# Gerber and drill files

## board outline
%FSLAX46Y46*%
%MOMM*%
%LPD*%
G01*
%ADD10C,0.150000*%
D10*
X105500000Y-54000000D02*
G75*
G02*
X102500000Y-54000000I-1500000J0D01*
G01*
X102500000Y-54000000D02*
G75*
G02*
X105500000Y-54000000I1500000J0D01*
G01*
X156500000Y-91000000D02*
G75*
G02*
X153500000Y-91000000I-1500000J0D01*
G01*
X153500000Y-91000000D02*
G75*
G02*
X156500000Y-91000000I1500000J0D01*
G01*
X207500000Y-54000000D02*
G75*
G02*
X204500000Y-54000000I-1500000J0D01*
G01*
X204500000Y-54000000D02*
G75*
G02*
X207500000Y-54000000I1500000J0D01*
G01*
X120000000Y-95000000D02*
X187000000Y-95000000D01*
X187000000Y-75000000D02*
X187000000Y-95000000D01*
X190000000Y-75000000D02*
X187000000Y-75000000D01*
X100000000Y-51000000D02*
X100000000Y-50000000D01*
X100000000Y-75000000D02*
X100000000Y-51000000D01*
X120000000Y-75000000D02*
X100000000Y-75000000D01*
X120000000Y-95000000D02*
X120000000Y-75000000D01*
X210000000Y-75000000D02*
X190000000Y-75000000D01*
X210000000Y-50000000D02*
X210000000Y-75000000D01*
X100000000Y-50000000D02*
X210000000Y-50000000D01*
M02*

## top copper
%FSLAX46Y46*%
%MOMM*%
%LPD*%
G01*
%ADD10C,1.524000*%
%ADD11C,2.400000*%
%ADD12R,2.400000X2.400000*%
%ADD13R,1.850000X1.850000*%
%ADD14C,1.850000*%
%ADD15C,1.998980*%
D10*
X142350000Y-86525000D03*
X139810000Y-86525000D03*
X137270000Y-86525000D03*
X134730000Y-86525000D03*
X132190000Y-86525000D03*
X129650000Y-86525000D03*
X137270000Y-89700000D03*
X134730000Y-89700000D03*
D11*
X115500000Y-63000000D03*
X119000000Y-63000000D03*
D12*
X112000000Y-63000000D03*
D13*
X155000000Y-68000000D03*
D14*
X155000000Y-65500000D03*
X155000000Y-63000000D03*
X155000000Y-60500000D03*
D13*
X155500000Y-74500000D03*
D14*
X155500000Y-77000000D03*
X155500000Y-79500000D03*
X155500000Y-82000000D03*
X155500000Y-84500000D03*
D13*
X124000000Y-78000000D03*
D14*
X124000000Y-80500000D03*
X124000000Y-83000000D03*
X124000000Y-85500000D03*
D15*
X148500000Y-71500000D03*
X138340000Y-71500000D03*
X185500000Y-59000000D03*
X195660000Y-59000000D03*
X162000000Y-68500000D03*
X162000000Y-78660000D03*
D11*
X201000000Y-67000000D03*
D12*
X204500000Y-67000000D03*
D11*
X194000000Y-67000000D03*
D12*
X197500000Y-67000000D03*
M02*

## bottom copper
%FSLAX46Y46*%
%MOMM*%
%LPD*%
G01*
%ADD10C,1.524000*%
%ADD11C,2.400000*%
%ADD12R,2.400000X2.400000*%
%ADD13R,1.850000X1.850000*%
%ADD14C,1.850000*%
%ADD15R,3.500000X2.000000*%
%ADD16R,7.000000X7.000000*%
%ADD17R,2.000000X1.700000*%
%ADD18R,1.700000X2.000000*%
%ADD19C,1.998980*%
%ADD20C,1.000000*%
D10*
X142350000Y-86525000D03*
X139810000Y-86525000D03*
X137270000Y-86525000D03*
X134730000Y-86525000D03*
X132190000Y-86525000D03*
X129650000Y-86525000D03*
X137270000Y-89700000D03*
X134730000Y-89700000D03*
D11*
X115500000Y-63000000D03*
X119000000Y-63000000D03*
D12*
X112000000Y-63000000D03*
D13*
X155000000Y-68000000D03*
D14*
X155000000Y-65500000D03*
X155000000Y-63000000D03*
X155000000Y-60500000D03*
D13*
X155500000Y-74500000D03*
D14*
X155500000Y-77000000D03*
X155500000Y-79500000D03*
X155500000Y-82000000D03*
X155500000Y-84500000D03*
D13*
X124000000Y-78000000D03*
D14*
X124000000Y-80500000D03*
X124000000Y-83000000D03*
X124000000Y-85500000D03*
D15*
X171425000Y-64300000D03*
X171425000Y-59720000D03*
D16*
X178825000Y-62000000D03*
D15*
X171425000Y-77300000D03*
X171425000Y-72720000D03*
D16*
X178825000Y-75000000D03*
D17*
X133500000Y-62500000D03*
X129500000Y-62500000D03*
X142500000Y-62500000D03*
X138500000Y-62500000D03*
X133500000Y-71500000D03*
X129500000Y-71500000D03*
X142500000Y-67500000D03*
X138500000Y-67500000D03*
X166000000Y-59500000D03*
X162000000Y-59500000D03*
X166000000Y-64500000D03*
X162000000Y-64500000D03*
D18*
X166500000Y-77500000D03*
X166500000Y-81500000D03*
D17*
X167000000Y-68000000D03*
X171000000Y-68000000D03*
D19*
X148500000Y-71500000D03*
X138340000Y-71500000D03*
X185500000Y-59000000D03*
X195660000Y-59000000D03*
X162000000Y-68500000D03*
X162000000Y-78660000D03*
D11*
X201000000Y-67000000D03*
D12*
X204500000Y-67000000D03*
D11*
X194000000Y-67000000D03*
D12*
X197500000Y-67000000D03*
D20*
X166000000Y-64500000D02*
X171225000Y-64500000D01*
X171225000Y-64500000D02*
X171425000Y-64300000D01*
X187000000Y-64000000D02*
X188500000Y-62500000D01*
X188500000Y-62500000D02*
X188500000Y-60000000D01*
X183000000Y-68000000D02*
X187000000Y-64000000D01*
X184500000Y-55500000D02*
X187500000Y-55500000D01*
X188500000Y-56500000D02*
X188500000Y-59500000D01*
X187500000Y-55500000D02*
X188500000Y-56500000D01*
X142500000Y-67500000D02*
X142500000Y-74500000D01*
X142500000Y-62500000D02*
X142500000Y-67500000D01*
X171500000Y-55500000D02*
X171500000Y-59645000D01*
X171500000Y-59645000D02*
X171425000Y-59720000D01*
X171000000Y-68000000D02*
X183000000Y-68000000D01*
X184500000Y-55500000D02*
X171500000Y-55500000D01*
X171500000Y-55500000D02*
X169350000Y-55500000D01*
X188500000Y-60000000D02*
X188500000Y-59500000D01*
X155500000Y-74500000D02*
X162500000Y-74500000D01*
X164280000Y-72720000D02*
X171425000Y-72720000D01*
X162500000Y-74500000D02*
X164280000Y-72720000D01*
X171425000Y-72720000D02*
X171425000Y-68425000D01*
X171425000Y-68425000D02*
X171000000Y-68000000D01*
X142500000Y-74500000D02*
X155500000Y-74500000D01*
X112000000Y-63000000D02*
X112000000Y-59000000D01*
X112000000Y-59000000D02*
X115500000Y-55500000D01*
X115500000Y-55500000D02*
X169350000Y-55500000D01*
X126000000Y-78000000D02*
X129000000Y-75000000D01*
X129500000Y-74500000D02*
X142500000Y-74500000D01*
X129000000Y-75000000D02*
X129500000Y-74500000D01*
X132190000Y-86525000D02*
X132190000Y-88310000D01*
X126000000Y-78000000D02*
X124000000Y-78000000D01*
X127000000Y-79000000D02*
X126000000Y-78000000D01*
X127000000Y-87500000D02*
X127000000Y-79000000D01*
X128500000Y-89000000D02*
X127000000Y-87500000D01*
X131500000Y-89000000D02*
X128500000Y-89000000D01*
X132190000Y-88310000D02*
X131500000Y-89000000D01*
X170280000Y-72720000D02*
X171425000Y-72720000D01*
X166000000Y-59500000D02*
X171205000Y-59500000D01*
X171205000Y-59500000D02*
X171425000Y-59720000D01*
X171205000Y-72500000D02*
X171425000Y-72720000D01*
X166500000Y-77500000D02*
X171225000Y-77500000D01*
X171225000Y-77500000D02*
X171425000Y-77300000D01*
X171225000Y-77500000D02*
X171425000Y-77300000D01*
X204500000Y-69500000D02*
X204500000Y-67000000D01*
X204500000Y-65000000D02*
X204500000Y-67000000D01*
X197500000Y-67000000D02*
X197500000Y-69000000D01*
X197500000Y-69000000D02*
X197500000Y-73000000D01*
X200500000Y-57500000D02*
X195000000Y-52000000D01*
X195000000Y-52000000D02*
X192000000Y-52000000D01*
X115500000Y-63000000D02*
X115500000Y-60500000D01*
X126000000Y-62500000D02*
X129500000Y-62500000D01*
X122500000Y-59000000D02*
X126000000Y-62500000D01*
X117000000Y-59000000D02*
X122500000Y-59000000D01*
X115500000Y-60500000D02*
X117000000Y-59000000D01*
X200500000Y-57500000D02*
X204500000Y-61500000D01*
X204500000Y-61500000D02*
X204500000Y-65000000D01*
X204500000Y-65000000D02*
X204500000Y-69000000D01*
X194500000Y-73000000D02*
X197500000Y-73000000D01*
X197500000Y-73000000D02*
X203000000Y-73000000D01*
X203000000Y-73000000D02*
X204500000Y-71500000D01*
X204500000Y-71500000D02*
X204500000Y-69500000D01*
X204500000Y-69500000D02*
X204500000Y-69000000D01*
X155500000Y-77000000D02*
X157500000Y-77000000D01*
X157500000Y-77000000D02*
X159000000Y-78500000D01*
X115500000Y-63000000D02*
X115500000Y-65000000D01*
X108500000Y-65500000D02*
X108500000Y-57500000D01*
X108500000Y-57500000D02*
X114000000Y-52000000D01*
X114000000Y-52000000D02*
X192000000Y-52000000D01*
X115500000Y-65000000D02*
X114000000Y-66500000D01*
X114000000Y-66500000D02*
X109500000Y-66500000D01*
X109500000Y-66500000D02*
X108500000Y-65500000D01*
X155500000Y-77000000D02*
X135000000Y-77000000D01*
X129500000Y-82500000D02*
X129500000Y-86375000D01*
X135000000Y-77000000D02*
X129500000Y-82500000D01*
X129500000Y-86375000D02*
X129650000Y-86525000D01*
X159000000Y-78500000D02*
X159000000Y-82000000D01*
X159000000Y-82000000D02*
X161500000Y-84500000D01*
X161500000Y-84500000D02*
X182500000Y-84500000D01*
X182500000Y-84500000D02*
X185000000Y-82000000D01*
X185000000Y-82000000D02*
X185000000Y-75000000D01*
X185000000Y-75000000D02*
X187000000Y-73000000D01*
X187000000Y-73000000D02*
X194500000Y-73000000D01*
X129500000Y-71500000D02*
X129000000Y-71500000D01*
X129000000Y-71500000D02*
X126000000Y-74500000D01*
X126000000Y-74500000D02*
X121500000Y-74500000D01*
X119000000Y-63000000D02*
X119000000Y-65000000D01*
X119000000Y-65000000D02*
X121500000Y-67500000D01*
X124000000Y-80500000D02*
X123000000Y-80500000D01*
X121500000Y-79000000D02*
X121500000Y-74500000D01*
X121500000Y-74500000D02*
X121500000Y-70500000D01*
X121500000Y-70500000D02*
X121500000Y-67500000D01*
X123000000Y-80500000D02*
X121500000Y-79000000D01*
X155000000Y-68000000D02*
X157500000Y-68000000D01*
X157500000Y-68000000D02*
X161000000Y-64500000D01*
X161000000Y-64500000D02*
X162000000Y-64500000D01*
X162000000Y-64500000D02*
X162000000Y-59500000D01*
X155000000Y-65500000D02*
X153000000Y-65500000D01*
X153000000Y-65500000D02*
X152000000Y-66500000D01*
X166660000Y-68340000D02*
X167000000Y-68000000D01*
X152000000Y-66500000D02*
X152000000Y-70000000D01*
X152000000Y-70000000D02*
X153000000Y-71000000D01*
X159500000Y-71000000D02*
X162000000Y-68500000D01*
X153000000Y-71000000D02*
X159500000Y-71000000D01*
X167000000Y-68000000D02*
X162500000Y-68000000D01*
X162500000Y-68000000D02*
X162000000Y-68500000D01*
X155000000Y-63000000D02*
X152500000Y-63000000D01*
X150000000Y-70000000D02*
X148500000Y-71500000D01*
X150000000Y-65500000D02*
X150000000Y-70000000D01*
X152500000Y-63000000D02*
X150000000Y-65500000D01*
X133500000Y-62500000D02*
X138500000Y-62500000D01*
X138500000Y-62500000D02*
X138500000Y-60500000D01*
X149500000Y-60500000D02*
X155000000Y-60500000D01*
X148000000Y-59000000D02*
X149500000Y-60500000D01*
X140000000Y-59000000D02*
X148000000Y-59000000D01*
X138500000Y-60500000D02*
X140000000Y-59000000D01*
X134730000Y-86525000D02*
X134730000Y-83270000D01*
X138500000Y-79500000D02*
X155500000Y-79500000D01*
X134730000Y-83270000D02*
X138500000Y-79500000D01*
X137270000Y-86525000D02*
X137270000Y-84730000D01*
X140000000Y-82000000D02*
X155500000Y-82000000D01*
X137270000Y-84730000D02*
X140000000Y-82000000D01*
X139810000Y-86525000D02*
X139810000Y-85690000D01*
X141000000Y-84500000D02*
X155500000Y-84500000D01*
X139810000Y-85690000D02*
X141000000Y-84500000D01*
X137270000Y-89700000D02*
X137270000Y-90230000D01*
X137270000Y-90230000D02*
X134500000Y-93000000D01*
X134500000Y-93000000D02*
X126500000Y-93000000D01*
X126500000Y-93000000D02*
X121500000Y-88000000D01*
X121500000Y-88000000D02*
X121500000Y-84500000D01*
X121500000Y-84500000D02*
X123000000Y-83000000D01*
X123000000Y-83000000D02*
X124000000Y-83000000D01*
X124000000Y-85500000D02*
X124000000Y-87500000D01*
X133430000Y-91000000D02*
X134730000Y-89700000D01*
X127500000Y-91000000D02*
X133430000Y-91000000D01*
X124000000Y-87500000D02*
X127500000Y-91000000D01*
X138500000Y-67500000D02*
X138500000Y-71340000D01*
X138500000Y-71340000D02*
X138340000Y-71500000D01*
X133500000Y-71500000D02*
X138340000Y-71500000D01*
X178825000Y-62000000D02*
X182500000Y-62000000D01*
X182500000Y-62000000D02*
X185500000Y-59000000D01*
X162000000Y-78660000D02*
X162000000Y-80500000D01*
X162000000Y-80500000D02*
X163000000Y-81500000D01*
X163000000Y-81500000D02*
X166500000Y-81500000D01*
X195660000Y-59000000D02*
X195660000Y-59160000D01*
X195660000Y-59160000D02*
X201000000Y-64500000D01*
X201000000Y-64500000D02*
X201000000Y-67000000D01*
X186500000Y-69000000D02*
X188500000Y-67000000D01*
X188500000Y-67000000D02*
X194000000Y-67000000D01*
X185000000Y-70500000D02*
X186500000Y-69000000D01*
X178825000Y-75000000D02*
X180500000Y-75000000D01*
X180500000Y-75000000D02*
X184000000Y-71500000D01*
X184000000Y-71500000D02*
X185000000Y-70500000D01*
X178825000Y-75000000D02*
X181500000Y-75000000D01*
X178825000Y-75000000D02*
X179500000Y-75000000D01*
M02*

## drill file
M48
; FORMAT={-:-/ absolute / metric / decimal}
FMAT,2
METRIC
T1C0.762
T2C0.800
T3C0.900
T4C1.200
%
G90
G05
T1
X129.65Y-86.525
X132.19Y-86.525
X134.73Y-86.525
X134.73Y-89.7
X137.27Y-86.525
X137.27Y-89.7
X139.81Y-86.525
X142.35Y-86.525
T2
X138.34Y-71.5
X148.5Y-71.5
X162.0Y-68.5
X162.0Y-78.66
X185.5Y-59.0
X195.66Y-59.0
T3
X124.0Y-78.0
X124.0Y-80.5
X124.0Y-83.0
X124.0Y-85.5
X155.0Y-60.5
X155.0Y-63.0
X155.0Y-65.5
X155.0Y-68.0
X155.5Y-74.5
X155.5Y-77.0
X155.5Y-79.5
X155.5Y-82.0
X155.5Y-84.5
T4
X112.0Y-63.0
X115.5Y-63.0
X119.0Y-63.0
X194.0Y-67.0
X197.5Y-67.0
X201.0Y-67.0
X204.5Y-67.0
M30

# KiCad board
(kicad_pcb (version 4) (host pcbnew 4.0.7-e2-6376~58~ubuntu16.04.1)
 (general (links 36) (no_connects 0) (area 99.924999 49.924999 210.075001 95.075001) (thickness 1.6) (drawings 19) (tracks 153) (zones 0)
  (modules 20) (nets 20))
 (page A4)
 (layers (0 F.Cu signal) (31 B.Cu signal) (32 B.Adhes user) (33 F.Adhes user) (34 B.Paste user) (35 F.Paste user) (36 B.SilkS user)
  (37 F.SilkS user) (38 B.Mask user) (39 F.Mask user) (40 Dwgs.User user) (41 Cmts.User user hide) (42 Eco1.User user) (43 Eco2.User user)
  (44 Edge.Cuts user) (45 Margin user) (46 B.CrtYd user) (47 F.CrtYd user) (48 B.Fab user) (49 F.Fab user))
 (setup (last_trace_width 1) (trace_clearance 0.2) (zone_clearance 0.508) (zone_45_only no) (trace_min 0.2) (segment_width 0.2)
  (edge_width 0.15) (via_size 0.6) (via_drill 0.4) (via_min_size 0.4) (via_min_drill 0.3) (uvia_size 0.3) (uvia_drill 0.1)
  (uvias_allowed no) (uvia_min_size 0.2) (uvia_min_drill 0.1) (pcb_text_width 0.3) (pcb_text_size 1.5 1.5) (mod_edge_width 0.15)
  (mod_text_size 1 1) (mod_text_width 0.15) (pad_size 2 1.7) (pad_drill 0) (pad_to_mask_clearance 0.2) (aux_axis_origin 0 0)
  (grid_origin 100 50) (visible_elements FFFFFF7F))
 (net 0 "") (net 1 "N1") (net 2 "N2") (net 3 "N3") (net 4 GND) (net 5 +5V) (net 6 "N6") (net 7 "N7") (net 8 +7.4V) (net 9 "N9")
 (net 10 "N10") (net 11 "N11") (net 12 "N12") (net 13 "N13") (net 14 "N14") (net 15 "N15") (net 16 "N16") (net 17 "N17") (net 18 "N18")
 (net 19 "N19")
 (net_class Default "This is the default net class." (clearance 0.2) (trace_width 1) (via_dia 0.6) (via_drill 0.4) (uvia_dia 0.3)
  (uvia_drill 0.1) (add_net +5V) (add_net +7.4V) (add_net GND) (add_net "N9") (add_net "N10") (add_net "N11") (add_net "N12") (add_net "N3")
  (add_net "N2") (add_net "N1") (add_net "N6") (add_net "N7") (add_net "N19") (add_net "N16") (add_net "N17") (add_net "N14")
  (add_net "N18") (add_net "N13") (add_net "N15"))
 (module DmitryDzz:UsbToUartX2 (layer F.Cu) (at 136 77)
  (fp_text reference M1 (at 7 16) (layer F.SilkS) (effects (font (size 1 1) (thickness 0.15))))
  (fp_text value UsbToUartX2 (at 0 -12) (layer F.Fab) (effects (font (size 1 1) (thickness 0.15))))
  (pad 1 thru_hole circle (at 6.35 9.525) (size 1.524 1.524) (drill 0.762) (layers *.Cu *.Mask))
  (pad 2 thru_hole circle (at 3.81 9.525) (size 1.524 1.524) (drill 0.762) (layers *.Cu *.Mask) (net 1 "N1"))
  (pad 3 thru_hole circle (at 1.27 9.525) (size 1.524 1.524) (drill 0.762) (layers *.Cu *.Mask) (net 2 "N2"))
  (pad 4 thru_hole circle (at -1.27 9.525) (size 1.524 1.524) (drill 0.762) (layers *.Cu *.Mask) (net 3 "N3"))
  (pad 5 thru_hole circle (at -3.81 9.525) (size 1.524 1.524) (drill 0.762) (layers *.Cu *.Mask) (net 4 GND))
  (pad 6 thru_hole circle (at -6.35 9.525) (size 1.524 1.524) (drill 0.762) (layers *.Cu *.Mask) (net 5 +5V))
  (pad 7 thru_hole circle (at 1.27 12.7) (size 1.524 1.524) (drill 0.762) (layers *.Cu *.Mask) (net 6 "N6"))
  (pad 8 thru_hole circle (at -1.27 12.7) (size 1.524 1.524) (drill 0.762) (layers *.Cu *.Mask) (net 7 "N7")))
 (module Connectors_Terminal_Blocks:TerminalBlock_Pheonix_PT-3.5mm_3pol (layer F.Cu) (at 112 63)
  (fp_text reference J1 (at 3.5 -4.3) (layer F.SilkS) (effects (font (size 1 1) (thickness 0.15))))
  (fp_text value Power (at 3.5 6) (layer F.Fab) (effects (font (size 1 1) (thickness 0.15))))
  (pad 2 thru_hole circle (at 3.5 0) (size 2.4 2.4) (drill 1.2) (layers *.Cu *.Mask) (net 5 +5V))
  (pad 3 thru_hole circle (at 7 0) (size 2.4 2.4) (drill 1.2) (layers *.Cu *.Mask) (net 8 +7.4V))
  (pad 1 thru_hole rect (at 0 0) (size 2.4 2.4) (drill 1.2) (layers *.Cu *.Mask) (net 4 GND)))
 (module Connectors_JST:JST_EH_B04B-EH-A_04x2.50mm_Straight (layer F.Cu) (at 155 68 90)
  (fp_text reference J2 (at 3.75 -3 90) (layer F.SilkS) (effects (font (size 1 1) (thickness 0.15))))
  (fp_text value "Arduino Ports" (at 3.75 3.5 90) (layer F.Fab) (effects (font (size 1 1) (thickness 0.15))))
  (pad 1 thru_hole rect (at 0 0 90) (size 1.85 1.85) (drill 0.9) (layers *.Cu *.Mask) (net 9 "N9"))
  (pad 2 thru_hole circle (at 2.5 0 90) (size 1.85 1.85) (drill 0.9) (layers *.Cu *.Mask) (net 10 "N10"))
  (pad 3 thru_hole circle (at 5 0 90) (size 1.85 1.85) (drill 0.9) (layers *.Cu *.Mask) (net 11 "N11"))
  (pad 4 thru_hole circle (at 7.5 0 90) (size 1.85 1.85) (drill 0.9) (layers *.Cu *.Mask) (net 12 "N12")))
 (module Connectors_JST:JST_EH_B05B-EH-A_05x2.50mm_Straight (layer F.Cu) (at 155.5 74.5 270)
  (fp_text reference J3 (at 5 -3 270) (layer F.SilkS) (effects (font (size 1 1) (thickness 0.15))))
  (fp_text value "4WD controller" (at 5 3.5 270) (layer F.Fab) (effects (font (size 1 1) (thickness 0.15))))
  (pad 1 thru_hole rect (at 0 0 270) (size 1.85 1.85) (drill 0.9) (layers *.Cu *.Mask) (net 4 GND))
  (pad 2 thru_hole circle (at 2.5 0 270) (size 1.85 1.85) (drill 0.9) (layers *.Cu *.Mask) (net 5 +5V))
  (pad 3 thru_hole circle (at 5 0 270) (size 1.85 1.85) (drill 0.9) (layers *.Cu *.Mask) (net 3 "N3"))
  (pad 4 thru_hole circle (at 7.5 0 270) (size 1.85 1.85) (drill 0.9) (layers *.Cu *.Mask) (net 2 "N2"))
  (pad 5 thru_hole circle (at 10 0 270) (size 1.85 1.85) (drill 0.9) (layers *.Cu *.Mask) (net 1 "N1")))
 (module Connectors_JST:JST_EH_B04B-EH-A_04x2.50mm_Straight (layer F.Cu) (at 124 78 270)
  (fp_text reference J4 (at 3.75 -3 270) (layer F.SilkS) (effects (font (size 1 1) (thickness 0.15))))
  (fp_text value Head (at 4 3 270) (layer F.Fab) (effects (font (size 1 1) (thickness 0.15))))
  (pad 1 thru_hole rect (at 0 0 270) (size 1.85 1.85) (drill 0.9) (layers *.Cu *.Mask) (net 4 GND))
  (pad 2 thru_hole circle (at 2.5 0 270) (size 1.85 1.85) (drill 0.9) (layers *.Cu *.Mask) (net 8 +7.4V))
  (pad 3 thru_hole circle (at 5 0 270) (size 1.85 1.85) (drill 0.9) (layers *.Cu *.Mask) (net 6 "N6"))
  (pad 4 thru_hole circle (at 7.5 0 270) (size 1.85 1.85) (drill 0.9) (layers *.Cu *.Mask) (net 7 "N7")))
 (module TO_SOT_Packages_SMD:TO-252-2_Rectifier (layer B.Cu) (at 176 62)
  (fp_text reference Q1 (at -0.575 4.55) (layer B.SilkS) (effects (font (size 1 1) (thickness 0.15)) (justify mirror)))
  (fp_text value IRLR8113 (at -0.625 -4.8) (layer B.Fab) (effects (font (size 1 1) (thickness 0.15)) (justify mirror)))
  (pad 1 smd rect (at -4.575 2.3 90) (size 2 3.5) (layers B.Cu B.Paste B.Mask) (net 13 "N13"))
  (pad 3 smd rect (at -4.575 -2.28 90) (size 2 3.5) (layers B.Cu B.Paste B.Mask) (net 4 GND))
  (pad 2 smd rect (at 2.825 0 90) (size 7 7) (layers B.Cu B.Paste B.Mask) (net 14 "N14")))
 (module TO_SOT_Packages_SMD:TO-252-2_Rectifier (layer B.Cu) (at 176 75)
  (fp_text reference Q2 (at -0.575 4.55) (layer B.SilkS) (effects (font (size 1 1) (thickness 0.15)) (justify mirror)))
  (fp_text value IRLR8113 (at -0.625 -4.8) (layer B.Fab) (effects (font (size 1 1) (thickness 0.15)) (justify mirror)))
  (pad 1 smd rect (at -4.575 2.3 90) (size 2 3.5) (layers B.Cu B.Paste B.Mask) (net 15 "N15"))
  (pad 3 smd rect (at -4.575 -2.28 90) (size 2 3.5) (layers B.Cu B.Paste B.Mask) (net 4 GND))
  (pad 2 smd rect (at 2.825 0 90) (size 7 7) (layers B.Cu B.Paste B.Mask) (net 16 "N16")))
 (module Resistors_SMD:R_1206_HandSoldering (layer B.Cu) (at 131.5 62.5 180)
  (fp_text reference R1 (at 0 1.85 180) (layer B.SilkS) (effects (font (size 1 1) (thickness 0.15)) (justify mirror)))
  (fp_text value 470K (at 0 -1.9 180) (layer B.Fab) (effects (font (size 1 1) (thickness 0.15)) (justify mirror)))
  (pad 1 smd rect (at -2 0 180) (size 2 1.7) (layers B.Cu B.Paste B.Mask) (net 12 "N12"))
  (pad 2 smd rect (at 2 0 180) (size 2 1.7) (layers B.Cu B.Paste B.Mask) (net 5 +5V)))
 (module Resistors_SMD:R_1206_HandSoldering (layer B.Cu) (at 140.5 62.5 180)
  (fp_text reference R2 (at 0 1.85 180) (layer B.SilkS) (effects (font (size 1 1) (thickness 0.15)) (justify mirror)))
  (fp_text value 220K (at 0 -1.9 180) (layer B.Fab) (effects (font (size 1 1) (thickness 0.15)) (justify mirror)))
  (pad 1 smd rect (at -2 0 180) (size 2 1.7) (layers B.Cu B.Paste B.Mask) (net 4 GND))
  (pad 2 smd rect (at 2 0 180) (size 2 1.7) (layers B.Cu B.Paste B.Mask) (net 12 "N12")))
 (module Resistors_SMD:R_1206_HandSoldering (layer B.Cu) (at 131.5 71.5 180)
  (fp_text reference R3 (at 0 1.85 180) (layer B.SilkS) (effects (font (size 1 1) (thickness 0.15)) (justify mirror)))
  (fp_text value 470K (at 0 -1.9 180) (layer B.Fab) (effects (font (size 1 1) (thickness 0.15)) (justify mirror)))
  (pad 1 smd rect (at -2 0 180) (size 2 1.7) (layers B.Cu B.Paste B.Mask) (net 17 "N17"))
  (pad 2 smd rect (at 2 0 180) (size 2 1.7) (layers B.Cu B.Paste B.Mask) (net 8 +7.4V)))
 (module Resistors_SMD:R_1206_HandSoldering (layer B.Cu) (at 140.5 67.5 180)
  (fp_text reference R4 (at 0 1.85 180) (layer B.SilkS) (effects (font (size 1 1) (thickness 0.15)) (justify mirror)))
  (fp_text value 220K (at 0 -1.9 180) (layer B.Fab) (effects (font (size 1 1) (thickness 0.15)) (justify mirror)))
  (pad 1 smd rect (at -2 0 180) (size 2 1.7) (layers B.Cu B.Paste B.Mask) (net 4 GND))
  (pad 2 smd rect (at 2 0 180) (size 2 1.7) (layers B.Cu B.Paste B.Mask) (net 17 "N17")))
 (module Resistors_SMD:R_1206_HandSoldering (layer B.Cu) (at 164 59.5 180)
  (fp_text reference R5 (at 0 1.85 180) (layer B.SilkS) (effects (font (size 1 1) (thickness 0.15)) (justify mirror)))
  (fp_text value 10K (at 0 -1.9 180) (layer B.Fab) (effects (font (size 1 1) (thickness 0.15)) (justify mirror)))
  (pad 1 smd rect (at -2 0 180) (size 2 1.7) (layers B.Cu B.Paste B.Mask) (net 4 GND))
  (pad 2 smd rect (at 2 0 180) (size 2 1.7) (layers B.Cu B.Paste B.Mask) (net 9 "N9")))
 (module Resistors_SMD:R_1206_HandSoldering (layer B.Cu) (at 164 64.5 180)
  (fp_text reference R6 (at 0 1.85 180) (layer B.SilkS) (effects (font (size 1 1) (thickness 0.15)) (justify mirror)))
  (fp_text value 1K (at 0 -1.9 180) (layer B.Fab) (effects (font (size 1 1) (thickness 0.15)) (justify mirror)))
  (pad 1 smd rect (at -2 0 180) (size 2 1.7) (layers B.Cu B.Paste B.Mask) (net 13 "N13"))
  (pad 2 smd rect (at 2 0 180) (size 2 1.7) (layers B.Cu B.Paste B.Mask) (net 9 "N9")))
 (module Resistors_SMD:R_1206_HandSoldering (layer B.Cu) (at 166.5 79.5 270)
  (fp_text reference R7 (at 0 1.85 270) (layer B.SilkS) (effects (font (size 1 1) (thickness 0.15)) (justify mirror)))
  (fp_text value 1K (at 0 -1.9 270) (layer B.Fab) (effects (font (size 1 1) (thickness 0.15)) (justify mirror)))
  (pad 1 smd rect (at -2 0 270) (size 2 1.7) (layers B.Cu B.Paste B.Mask) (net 15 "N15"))
  (pad 2 smd rect (at 2 0 270) (size 2 1.7) (layers B.Cu B.Paste B.Mask) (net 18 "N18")))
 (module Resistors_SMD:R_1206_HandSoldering (layer B.Cu) (at 169 68)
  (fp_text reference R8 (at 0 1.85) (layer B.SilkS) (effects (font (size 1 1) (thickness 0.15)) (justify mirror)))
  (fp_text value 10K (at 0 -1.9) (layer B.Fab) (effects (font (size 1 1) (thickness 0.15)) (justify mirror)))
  (pad 1 smd rect (at -2 0) (size 2 1.7) (layers B.Cu B.Paste B.Mask) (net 10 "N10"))
  (pad 2 smd rect (at 2 0) (size 2 1.7) (layers B.Cu B.Paste B.Mask) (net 4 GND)))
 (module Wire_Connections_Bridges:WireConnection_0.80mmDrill (layer F.Cu) (at 148.5 71.5 180)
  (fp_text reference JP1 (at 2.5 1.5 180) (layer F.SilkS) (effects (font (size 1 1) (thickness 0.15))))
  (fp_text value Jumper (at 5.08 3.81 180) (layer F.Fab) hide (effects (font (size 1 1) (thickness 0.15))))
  (pad 1 thru_hole circle (at 0 0 180) (size 1.99898 1.99898) (drill 0.8001) (layers *.Cu *.Mask) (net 11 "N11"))
  (pad 2 thru_hole circle (at 10.16 0 180) (size 1.99898 1.99898) (drill 0.8001) (layers *.Cu *.Mask) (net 17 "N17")))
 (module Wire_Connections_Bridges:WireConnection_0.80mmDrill (layer F.Cu) (at 185.5 59)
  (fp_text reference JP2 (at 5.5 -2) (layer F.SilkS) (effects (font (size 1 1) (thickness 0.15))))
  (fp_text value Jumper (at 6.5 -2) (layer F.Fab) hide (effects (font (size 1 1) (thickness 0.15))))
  (pad 1 thru_hole circle (at 0 0) (size 1.99898 1.99898) (drill 0.8001) (layers *.Cu *.Mask) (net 14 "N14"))
  (pad 2 thru_hole circle (at 10.16 0) (size 1.99898 1.99898) (drill 0.8001) (layers *.Cu *.Mask) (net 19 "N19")))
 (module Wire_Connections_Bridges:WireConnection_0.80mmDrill (layer F.Cu) (at 162 68.5 270)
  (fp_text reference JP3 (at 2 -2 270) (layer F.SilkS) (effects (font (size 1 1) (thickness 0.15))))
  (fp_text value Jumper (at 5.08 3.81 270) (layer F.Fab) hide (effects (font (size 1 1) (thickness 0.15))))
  (pad 1 thru_hole circle (at 0 0 270) (size 1.99898 1.99898) (drill 0.8001) (layers *.Cu *.Mask) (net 10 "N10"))
  (pad 2 thru_hole circle (at 10.16 0 270) (size 1.99898 1.99898) (drill 0.8001) (layers *.Cu *.Mask) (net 18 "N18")))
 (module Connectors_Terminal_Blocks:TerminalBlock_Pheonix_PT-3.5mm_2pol (layer F.Cu) (at 204.5 67 180)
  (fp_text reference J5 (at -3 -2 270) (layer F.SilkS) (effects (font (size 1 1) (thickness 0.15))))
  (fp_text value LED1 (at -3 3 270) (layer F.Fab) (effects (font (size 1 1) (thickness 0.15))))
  (pad 2 thru_hole circle (at 3.5 0 180) (size 2.4 2.4) (drill 1.2) (layers *.Cu *.Mask) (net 19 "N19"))
  (pad 1 thru_hole rect (at 0 0 180) (size 2.4 2.4) (drill 1.2) (layers *.Cu *.Mask) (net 5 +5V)))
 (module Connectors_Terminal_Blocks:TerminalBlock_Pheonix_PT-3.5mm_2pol (layer F.Cu) (at 197.5 67 180)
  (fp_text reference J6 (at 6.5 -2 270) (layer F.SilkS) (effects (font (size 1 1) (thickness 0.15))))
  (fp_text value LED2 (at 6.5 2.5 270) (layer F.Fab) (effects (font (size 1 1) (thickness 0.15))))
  (pad 2 thru_hole circle (at 3.5 0 180) (size 2.4 2.4) (drill 1.2) (layers *.Cu *.Mask) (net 16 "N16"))
  (pad 1 thru_hole rect (at 0 0 180) (size 2.4 2.4) (drill 1.2) (layers *.Cu *.Mask) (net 5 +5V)))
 (gr_circle (center 104 54) (end 105.5 54) (layer Edge.Cuts) (width 0.15))
 (gr_circle (center 155 91) (end 156.5 91) (layer Edge.Cuts) (width 0.15))
 (gr_circle (center 206 54) (end 207.5 54) (layer Edge.Cuts) (width 0.15))
 (gr_line (start 120 95) (end 187 95) (angle 90) (layer Edge.Cuts) (width 0.15))
 (gr_line (start 187 75) (end 187 95) (angle 90) (layer Edge.Cuts) (width 0.15))
 (gr_line (start 190 75) (end 187 75) (angle 90) (layer Edge.Cuts) (width 0.15))
 (gr_line (start 100 51) (end 100 50) (angle 90) (layer Edge.Cuts) (width 0.15))
 (gr_line (start 100 75) (end 100 51) (angle 90) (layer Edge.Cuts) (width 0.15))
 (gr_line (start 120 75) (end 100 75) (angle 90) (layer Edge.Cuts) (width 0.15))
 (gr_line (start 120 95) (end 120 75) (angle 90) (layer Edge.Cuts) (width 0.15))
 (gr_line (start 210 75) (end 190 75) (angle 90) (layer Edge.Cuts) (width 0.15))
 (gr_line (start 210 50) (end 210 75) (angle 90) (layer Edge.Cuts) (width 0.15))
 (gr_line (start 100 50) (end 210 50) (angle 90) (layer Edge.Cuts) (width 0.15))
 (segment (start 166 64.5) (end 171.225 64.5) (width 1) (layer B.Cu) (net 13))
 (segment (start 171.225 64.5) (end 171.425 64.3) (width 1) (layer B.Cu) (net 13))
 (segment (start 187 64) (end 188.5 62.5) (width 1) (layer B.Cu) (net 4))
 (segment (start 188.5 62.5) (end 188.5 60) (width 1) (layer B.Cu) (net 4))
 (segment (start 183 68) (end 187 64) (width 1) (layer B.Cu) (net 4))
 (segment (start 184.5 55.5) (end 187.5 55.5) (width 1) (layer B.Cu) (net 4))
 (segment (start 188.5 56.5) (end 188.5 59.5) (width 1) (layer B.Cu) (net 4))
 (segment (start 187.5 55.5) (end 188.5 56.5) (width 1) (layer B.Cu) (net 4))
 (segment (start 142.5 67.5) (end 142.5 74.5) (width 1) (layer B.Cu) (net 4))
 (segment (start 142.5 62.5) (end 142.5 67.5) (width 1) (layer B.Cu) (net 4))
 (segment (start 171.5 55.5) (end 171.5 59.645) (width 1) (layer B.Cu) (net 4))
 (segment (start 171.5 59.645) (end 171.425 59.72) (width 1) (layer B.Cu) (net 4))
 (segment (start 171 68) (end 183 68) (width 1) (layer B.Cu) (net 4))
 (segment (start 184.5 55.5) (end 171.5 55.5) (width 1) (layer B.Cu) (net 4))
 (segment (start 171.5 55.5) (end 169.35 55.5) (width 1) (layer B.Cu) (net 4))
 (segment (start 188.5 60) (end 188.5 59.5) (width 1) (layer B.Cu) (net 4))
 (segment (start 155.5 74.5) (end 162.5 74.5) (width 1) (layer B.Cu) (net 4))
 (segment (start 164.28 72.72) (end 171.425 72.72) (width 1) (layer B.Cu) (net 4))
 (segment (start 162.5 74.5) (end 164.28 72.72) (width 1) (layer B.Cu) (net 4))
 (segment (start 171.425 72.72) (end 171.425 68.425) (width 1) (layer B.Cu) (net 4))
 (segment (start 171.425 68.425) (end 171 68) (width 1) (layer B.Cu) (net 4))
 (segment (start 142.5 74.5) (end 155.5 74.5) (width 1) (layer B.Cu) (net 4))
 (segment (start 112 63) (end 112 59) (width 1) (layer B.Cu) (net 4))
 (segment (start 112 59) (end 115.5 55.5) (width 1) (layer B.Cu) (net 4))
 (segment (start 115.5 55.5) (end 169.35 55.5) (width 1) (layer B.Cu) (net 4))
 (segment (start 126 78) (end 129 75) (width 1) (layer B.Cu) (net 4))
 (segment (start 129.5 74.5) (end 142.5 74.5) (width 1) (layer B.Cu) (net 4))
 (segment (start 129 75) (end 129.5 74.5) (width 1) (layer B.Cu) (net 4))
 (segment (start 132.19 86.525) (end 132.19 88.31) (width 1) (layer B.Cu) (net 4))
 (segment (start 126 78) (end 124 78) (width 1) (layer B.Cu) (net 4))
 (segment (start 127 79) (end 126 78) (width 1) (layer B.Cu) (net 4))
 (segment (start 127 87.5) (end 127 79) (width 1) (layer B.Cu) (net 4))
 (segment (start 128.5 89) (end 127 87.5) (width 1) (layer B.Cu) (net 4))
 (segment (start 131.5 89) (end 128.5 89) (width 1) (layer B.Cu) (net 4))
 (segment (start 132.19 88.31) (end 131.5 89) (width 1) (layer B.Cu) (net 4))
 (segment (start 170.28 72.72) (end 171.425 72.72) (width 1) (layer B.Cu) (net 4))
 (segment (start 166 59.5) (end 171.205 59.5) (width 1) (layer B.Cu) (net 4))
 (segment (start 171.205 59.5) (end 171.425 59.72) (width 1) (layer B.Cu) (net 4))
 (segment (start 171.205 72.5) (end 171.425 72.72) (width 1) (layer B.Cu) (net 4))
 (segment (start 166.5 77.5) (end 171.225 77.5) (width 1) (layer B.Cu) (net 15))
 (segment (start 171.225 77.5) (end 171.425 77.3) (width 1) (layer B.Cu) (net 15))
 (segment (start 171.225 77.5) (end 171.425 77.3) (width 1) (layer B.Cu) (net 15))
 (segment (start 204.5 69.5) (end 204.5 67) (width 1) (layer B.Cu) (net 5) (status 800000))
 (segment (start 204.5 65) (end 204.5 67) (width 1) (layer B.Cu) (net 5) (status 800000))
 (segment (start 197.5 67) (end 197.5 69) (width 1) (layer B.Cu) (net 5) (status 400000))
 (segment (start 197.5 69) (end 197.5 73) (width 1) (layer B.Cu) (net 5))
 (segment (start 200.5 57.5) (end 195 52) (width 1) (layer B.Cu) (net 5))
 (segment (start 195 52) (end 192 52) (width 1) (layer B.Cu) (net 5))
 (segment (start 115.5 63) (end 115.5 60.5) (width 1) (layer B.Cu) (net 5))
 (segment (start 126 62.5) (end 129.5 62.5) (width 1) (layer B.Cu) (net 5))
 (segment (start 122.5 59) (end 126 62.5) (width 1) (layer B.Cu) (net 5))
 (segment (start 117 59) (end 122.5 59) (width 1) (layer B.Cu) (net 5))
 (segment (start 115.5 60.5) (end 117 59) (width 1) (layer B.Cu) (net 5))
 (segment (start 200.5 57.5) (end 204.5 61.5) (width 1) (layer B.Cu) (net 5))
 (segment (start 204.5 61.5) (end 204.5 65) (width 1) (layer B.Cu) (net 5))
 (segment (start 204.5 65) (end 204.5 69) (width 1) (layer B.Cu) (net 5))
 (segment (start 194.5 73) (end 197.5 73) (width 1) (layer B.Cu) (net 5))
 (segment (start 197.5 73) (end 203 73) (width 1) (layer B.Cu) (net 5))
 (segment (start 203 73) (end 204.5 71.5) (width 1) (layer B.Cu) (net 5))
 (segment (start 204.5 71.5) (end 204.5 69.5) (width 1) (layer B.Cu) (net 5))
 (segment (start 204.5 69.5) (end 204.5 69) (width 1) (layer B.Cu) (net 5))
 (segment (start 155.5 77) (end 157.5 77) (width 1) (layer B.Cu) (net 5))
 (segment (start 157.5 77) (end 159 78.5) (width 1) (layer B.Cu) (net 5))
 (segment (start 115.5 63) (end 115.5 65) (width 1) (layer B.Cu) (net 5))
 (segment (start 108.5 65.5) (end 108.5 57.5) (width 1) (layer B.Cu) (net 5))
 (segment (start 108.5 57.5) (end 114 52) (width 1) (layer B.Cu) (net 5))
 (segment (start 114 52) (end 192 52) (width 1) (layer B.Cu) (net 5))
 (segment (start 115.5 65) (end 114 66.5) (width 1) (layer B.Cu) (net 5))
 (segment (start 114 66.5) (end 109.5 66.5) (width 1) (layer B.Cu) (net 5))
 (segment (start 109.5 66.5) (end 108.5 65.5) (width 1) (layer B.Cu) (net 5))
 (segment (start 155.5 77) (end 135 77) (width 1) (layer B.Cu) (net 5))
 (segment (start 129.5 82.5) (end 129.5 86.375) (width 1) (layer B.Cu) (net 5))
 (segment (start 135 77) (end 129.5 82.5) (width 1) (layer B.Cu) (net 5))
 (segment (start 129.5 86.375) (end 129.65 86.525) (width 1) (layer B.Cu) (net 5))
 (segment (start 159 78.5) (end 159 82) (width 1) (layer B.Cu) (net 5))
 (segment (start 159 82) (end 161.5 84.5) (width 1) (layer B.Cu) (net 5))
 (segment (start 161.5 84.5) (end 182.5 84.5) (width 1) (layer B.Cu) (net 5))
 (segment (start 182.5 84.5) (end 185 82) (width 1) (layer B.Cu) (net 5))
 (segment (start 185 82) (end 185 75) (width 1) (layer B.Cu) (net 5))
 (segment (start 185 75) (end 187 73) (width 1) (layer B.Cu) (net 5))
 (segment (start 187 73) (end 194.5 73) (width 1) (layer B.Cu) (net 5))
 (segment (start 129.5 71.5) (end 129 71.5) (width 1) (layer B.Cu) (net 8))
 (segment (start 129 71.5) (end 126 74.5) (width 1) (layer B.Cu) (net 8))
 (segment (start 126 74.5) (end 121.5 74.5) (width 1) (layer B.Cu) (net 8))
 (segment (start 119 63) (end 119 65) (width 1) (layer B.Cu) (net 8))
 (segment (start 119 65) (end 121.5 67.5) (width 1) (layer B.Cu) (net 8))
 (segment (start 124 80.5) (end 123 80.5) (width 1) (layer B.Cu) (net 8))
 (segment (start 121.5 79) (end 121.5 74.5) (width 1) (layer B.Cu) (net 8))
 (segment (start 121.5 74.5) (end 121.5 70.5) (width 1) (layer B.Cu) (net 8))
 (segment (start 121.5 70.5) (end 121.5 67.5) (width 1) (layer B.Cu) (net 8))
 (segment (start 123 80.5) (end 121.5 79) (width 1) (layer B.Cu) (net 8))
 (segment (start 155 68) (end 157.5 68) (width 1) (layer B.Cu) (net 9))
 (segment (start 157.5 68) (end 161 64.5) (width 1) (layer B.Cu) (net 9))
 (segment (start 161 64.5) (end 162 64.5) (width 1) (layer B.Cu) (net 9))
 (segment (start 162 64.5) (end 162 59.5) (width 1) (layer B.Cu) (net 9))
 (segment (start 155 65.5) (end 153 65.5) (width 1) (layer B.Cu) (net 10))
 (segment (start 153 65.5) (end 152 66.5) (width 1) (layer B.Cu) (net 10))
 (segment (start 166.66 68.34) (end 167 68) (width 1) (layer B.Cu) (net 10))
 (segment (start 152 66.5) (end 152 70) (width 1) (layer B.Cu) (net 10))
 (segment (start 152 70) (end 153 71) (width 1) (layer B.Cu) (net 10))
 (segment (start 159.5 71) (end 162 68.5) (width 1) (layer B.Cu) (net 10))
 (segment (start 153 71) (end 159.5 71) (width 1) (layer B.Cu) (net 10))
 (segment (start 167 68) (end 162.5 68) (width 1) (layer B.Cu) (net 10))
 (segment (start 162.5 68) (end 162 68.5) (width 1) (layer B.Cu) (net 10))
 (segment (start 155 63) (end 152.5 63) (width 1) (layer B.Cu) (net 11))
 (segment (start 150 70) (end 148.5 71.5) (width 1) (layer B.Cu) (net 11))
 (segment (start 150 65.5) (end 150 70) (width 1) (layer B.Cu) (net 11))
 (segment (start 152.5 63) (end 150 65.5) (width 1) (layer B.Cu) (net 11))
 (segment (start 133.5 62.5) (end 138.5 62.5) (width 1) (layer B.Cu) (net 12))
 (segment (start 138.5 62.5) (end 138.5 60.5) (width 1) (layer B.Cu) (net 12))
 (segment (start 149.5 60.5) (end 155 60.5) (width 1) (layer B.Cu) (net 12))
 (segment (start 148 59) (end 149.5 60.5) (width 1) (layer B.Cu) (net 12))
 (segment (start 140 59) (end 148 59) (width 1) (layer B.Cu) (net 12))
 (segment (start 138.5 60.5) (end 140 59) (width 1) (layer B.Cu) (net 12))
 (segment (start 134.73 86.525) (end 134.73 83.27) (width 1) (layer B.Cu) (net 3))
 (segment (start 138.5 79.5) (end 155.5 79.5) (width 1) (layer B.Cu) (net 3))
 (segment (start 134.73 83.27) (end 138.5 79.5) (width 1) (layer B.Cu) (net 3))
 (segment (start 137.27 86.525) (end 137.27 84.73) (width 1) (layer B.Cu) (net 2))
 (segment (start 140 82) (end 155.5 82) (width 1) (layer B.Cu) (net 2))
 (segment (start 137.27 84.73) (end 140 82) (width 1) (layer B.Cu) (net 2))
 (segment (start 139.81 86.525) (end 139.81 85.69) (width 1) (layer B.Cu) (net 1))
 (segment (start 141 84.5) (end 155.5 84.5) (width 1) (layer B.Cu) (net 1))
 (segment (start 139.81 85.69) (end 141 84.5) (width 1) (layer B.Cu) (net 1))
 (segment (start 137.27 89.7) (end 137.27 90.23) (width 1) (layer B.Cu) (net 6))
 (segment (start 137.27 90.23) (end 134.5 93) (width 1) (layer B.Cu) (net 6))
 (segment (start 134.5 93) (end 126.5 93) (width 1) (layer B.Cu) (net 6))
 (segment (start 126.5 93) (end 121.5 88) (width 1) (layer B.Cu) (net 6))
 (segment (start 121.5 88) (end 121.5 84.5) (width 1) (layer B.Cu) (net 6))
 (segment (start 121.5 84.5) (end 123 83) (width 1) (layer B.Cu) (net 6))
 (segment (start 123 83) (end 124 83) (width 1) (layer B.Cu) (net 6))
 (segment (start 124 85.5) (end 124 87.5) (width 1) (layer B.Cu) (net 7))
 (segment (start 133.43 91) (end 134.73 89.7) (width 1) (layer B.Cu) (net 7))
 (segment (start 127.5 91) (end 133.43 91) (width 1) (layer B.Cu) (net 7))
 (segment (start 124 87.5) (end 127.5 91) (width 1) (layer B.Cu) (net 7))
 (segment (start 138.5 67.5) (end 138.5 71.34) (width 1) (layer B.Cu) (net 17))
 (segment (start 138.5 71.34) (end 138.34 71.5) (width 1) (layer B.Cu) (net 17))
 (segment (start 133.5 71.5) (end 138.34 71.5) (width 1) (layer B.Cu) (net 17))
 (segment (start 178.825 62) (end 182.5 62) (width 1) (layer B.Cu) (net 14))
 (segment (start 182.5 62) (end 185.5 59) (width 1) (layer B.Cu) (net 14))
 (segment (start 162 78.66) (end 162 80.5) (width 1) (layer B.Cu) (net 18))
 (segment (start 162 80.5) (end 163 81.5) (width 1) (layer B.Cu) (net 18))
 (segment (start 163 81.5) (end 166.5 81.5) (width 1) (layer B.Cu) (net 18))
 (segment (start 195.66 59) (end 195.66 59.16) (width 1) (layer B.Cu) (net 19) (status C00000))
 (segment (start 195.66 59.16) (end 201 64.5) (width 1) (layer B.Cu) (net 19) (status 400000))
 (segment (start 201 64.5) (end 201 67) (width 1) (layer B.Cu) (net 19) (status 800000))
 (segment (start 186.5 69) (end 188.5 67) (width 1) (layer B.Cu) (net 16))
 (segment (start 188.5 67) (end 194 67) (width 1) (layer B.Cu) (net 16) (status 800000))
 (segment (start 185 70.5) (end 186.5 69) (width 1) (layer B.Cu) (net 16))
 (segment (start 178.825 75) (end 180.5 75) (width 1) (layer B.Cu) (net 16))
 (segment (start 180.5 75) (end 184 71.5) (width 1) (layer B.Cu) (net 16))
 (segment (start 184 71.5) (end 185 70.5) (width 1) (layer B.Cu) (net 16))
 (segment (start 178.825 75) (end 181.5 75) (width 1) (layer B.Cu) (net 16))
 (segment (start 178.825 75) (end 179.5 75) (width 1) (layer B.Cu) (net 16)))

